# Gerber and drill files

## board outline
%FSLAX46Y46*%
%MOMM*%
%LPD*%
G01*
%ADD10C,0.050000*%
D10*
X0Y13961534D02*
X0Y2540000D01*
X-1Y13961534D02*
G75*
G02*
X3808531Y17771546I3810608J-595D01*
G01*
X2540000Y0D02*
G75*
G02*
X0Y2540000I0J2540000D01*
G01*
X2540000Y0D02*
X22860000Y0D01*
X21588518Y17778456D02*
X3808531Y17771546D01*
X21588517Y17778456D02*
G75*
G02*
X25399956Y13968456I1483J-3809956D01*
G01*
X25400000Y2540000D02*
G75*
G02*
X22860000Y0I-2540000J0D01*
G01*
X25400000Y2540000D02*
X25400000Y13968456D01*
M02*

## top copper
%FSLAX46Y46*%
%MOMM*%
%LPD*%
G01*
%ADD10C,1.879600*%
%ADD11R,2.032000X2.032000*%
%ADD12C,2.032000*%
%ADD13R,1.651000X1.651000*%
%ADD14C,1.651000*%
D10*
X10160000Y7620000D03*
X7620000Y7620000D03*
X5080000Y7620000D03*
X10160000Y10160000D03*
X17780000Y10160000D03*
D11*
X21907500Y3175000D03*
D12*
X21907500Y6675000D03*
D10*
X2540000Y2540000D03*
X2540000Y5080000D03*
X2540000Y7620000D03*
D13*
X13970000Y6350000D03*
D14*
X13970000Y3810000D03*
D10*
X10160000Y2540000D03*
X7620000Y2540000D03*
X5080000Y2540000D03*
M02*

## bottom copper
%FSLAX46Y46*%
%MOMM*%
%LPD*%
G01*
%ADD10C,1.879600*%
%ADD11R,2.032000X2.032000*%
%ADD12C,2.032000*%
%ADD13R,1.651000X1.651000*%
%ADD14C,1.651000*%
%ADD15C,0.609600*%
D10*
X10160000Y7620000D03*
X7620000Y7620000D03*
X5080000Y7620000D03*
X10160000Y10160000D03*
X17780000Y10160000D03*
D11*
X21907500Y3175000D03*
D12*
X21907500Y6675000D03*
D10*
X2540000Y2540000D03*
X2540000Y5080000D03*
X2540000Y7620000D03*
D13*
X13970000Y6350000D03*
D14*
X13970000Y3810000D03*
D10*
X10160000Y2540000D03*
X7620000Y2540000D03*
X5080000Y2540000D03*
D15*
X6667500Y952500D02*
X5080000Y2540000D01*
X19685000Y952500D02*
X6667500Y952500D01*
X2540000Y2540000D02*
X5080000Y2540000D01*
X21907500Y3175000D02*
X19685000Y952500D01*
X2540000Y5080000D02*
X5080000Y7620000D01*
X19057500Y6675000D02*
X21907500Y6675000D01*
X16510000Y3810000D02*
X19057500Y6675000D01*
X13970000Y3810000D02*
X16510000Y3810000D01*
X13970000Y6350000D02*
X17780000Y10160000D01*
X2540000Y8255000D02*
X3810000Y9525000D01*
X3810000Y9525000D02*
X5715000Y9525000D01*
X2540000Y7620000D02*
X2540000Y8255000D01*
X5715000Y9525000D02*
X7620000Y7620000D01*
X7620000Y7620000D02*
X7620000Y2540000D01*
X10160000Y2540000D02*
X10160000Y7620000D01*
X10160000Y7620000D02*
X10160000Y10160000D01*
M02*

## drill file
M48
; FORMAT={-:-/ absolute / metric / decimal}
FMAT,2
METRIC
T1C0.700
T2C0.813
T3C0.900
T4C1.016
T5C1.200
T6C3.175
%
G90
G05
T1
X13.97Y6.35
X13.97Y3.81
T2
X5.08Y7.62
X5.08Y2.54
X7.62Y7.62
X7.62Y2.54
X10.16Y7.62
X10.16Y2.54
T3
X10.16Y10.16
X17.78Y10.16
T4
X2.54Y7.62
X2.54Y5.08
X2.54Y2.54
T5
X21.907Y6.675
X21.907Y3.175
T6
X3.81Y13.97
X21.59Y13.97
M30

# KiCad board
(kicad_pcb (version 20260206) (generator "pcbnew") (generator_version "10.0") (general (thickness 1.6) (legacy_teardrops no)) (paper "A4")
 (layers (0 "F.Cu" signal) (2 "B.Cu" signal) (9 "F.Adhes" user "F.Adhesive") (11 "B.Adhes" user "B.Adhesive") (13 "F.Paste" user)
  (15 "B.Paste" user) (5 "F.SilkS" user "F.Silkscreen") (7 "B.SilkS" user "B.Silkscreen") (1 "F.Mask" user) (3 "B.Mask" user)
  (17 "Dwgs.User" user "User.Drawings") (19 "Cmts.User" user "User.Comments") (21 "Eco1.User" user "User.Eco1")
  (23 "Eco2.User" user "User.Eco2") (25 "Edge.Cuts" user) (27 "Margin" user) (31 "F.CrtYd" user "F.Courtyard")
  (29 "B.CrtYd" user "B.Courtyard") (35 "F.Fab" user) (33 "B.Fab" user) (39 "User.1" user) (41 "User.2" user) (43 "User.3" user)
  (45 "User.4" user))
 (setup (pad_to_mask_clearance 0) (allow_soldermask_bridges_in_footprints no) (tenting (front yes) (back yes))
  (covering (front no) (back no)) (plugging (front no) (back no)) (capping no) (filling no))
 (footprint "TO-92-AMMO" (layer "F.Cu") (at 7.62 -7.62 180)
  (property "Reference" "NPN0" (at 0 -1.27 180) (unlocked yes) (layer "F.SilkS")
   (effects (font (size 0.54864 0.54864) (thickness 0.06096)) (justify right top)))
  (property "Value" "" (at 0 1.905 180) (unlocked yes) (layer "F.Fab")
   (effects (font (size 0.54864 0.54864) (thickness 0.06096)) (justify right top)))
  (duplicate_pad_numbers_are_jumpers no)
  (pad "1" thru_hole circle (at -2.54 0 180) (size 1.8796 1.8796) (drill 0.8128) (layers "*.Cu" "*.Mask") (remove_unused_layers no)
   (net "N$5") (solder_mask_margin 0.1016) (thermal_bridge_angle 0))
  (pad "2" thru_hole circle (at 0 0 180) (size 1.8796 1.8796) (drill 0.8128) (layers "*.Cu" "*.Mask") (remove_unused_layers no) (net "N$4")
   (solder_mask_margin 0.1016) (thermal_bridge_angle 0))
  (pad "3" thru_hole circle (at 2.54 0 180) (size 1.8796 1.8796) (drill 0.8128) (layers "*.Cu" "*.Mask") (remove_unused_layers no)
   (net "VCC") (solder_mask_margin 0.1016) (thermal_bridge_angle 0)))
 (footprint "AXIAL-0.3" (layer "F.Cu") (at 13.97 -10.16)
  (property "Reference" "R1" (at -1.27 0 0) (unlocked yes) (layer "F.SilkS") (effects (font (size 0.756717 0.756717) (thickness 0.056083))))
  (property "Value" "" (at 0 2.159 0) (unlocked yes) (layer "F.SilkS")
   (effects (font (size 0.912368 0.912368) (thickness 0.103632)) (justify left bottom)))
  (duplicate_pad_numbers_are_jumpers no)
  (pad "P$1" thru_hole circle (at -3.81 0) (size 1.8796 1.8796) (drill 0.9) (layers "*.Cu" "*.Mask") (remove_unused_layers no) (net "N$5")
   (solder_mask_margin 0.1016) (thermal_bridge_angle 0))
  (pad "P$2" thru_hole circle (at 3.81 0) (size 1.8796 1.8796) (drill 0.9) (layers "*.Cu" "*.Mask") (remove_unused_layers no) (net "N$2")
   (solder_mask_margin 0.1016) (thermal_bridge_angle 0)))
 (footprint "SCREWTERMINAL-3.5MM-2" (layer "F.Cu") (at 21.9075 -3.175 90)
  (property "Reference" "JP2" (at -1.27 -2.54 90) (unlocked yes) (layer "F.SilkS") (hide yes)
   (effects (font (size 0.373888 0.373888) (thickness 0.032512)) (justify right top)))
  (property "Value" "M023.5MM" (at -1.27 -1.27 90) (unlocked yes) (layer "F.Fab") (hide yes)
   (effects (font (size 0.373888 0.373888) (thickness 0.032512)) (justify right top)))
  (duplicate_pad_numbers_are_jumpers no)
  (pad "1" thru_hole rect (at 0 0 90) (size 2.032 2.032) (drill 1.2) (layers "*.Cu" "*.Mask") (remove_unused_layers no) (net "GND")
   (solder_mask_margin 0.1016) (thermal_bridge_angle 0))
  (pad "2" thru_hole circle (at 3.5 0 90) (size 2.032 2.032) (drill 1.2) (layers "*.Cu" "*.Mask") (remove_unused_layers no) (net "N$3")
   (solder_mask_margin 0.1016) (thermal_bridge_angle 0)))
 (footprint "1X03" (layer "F.Cu") (at 2.54 -2.54 90)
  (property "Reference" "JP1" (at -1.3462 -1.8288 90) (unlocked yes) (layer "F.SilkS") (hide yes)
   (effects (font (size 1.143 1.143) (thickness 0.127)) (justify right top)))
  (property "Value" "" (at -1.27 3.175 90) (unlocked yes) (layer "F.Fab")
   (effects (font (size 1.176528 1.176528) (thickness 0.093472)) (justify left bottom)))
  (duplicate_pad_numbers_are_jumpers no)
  (pad "1" thru_hole circle (at 0 0 180) (size 1.8796 1.8796) (drill 1.016) (layers "*.Cu" "*.Mask") (remove_unused_layers no) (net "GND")
   (solder_mask_margin 0.1016) (thermal_bridge_angle 0))
  (pad "2" thru_hole circle (at 2.54 0 180) (size 1.8796 1.8796) (drill 1.016) (layers "*.Cu" "*.Mask") (remove_unused_layers no)
   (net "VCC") (solder_mask_margin 0.1016) (thermal_bridge_angle 0))
  (pad "3" thru_hole circle (at 5.08 0 180) (size 1.8796 1.8796) (drill 1.016) (layers "*.Cu" "*.Mask") (remove_unused_layers no)
   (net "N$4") (solder_mask_margin 0.1016) (thermal_bridge_angle 0)))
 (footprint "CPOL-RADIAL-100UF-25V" (layer "F.Cu") (at 13.97 -5.08 90)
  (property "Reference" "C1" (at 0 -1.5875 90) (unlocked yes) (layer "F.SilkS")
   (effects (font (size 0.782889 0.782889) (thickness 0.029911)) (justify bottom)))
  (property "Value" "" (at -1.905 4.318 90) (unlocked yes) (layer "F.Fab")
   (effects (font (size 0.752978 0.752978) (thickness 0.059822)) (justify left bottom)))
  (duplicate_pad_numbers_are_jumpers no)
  (pad "1" thru_hole rect (at 1.27 0 90) (size 1.651 1.651) (drill 0.7) (layers "*.Cu" "*.Mask") (remove_unused_layers no) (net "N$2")
   (solder_mask_margin 0.1016) (thermal_bridge_angle 0))
  (pad "2" thru_hole circle (at -1.27 0 90) (size 1.651 1.651) (drill 0.7) (layers "*.Cu" "*.Mask") (remove_unused_layers no) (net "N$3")
   (solder_mask_margin 0.1016) (thermal_bridge_angle 0)))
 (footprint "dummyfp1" (layer "F.Cu") (at 21.59 -13.97)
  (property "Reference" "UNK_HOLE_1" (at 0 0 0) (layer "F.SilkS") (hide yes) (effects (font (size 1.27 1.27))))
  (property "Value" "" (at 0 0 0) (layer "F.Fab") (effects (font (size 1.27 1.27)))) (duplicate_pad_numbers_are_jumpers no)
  (pad "" np_thru_hole circle (at 0 0) (size 3.175 3.175) (drill 3.175) (layers "*.Cu" "*.Mask")))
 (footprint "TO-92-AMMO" (layer "F.Cu") (at 7.62 -2.54 180)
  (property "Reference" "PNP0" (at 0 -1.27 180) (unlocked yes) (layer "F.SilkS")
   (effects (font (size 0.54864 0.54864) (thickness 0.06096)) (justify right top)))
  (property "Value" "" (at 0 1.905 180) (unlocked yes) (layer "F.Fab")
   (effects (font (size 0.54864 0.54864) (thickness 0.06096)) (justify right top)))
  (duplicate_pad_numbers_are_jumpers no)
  (pad "1" thru_hole circle (at -2.54 0 180) (size 1.8796 1.8796) (drill 0.8128) (layers "*.Cu" "*.Mask") (remove_unused_layers no)
   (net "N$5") (solder_mask_margin 0.1016) (thermal_bridge_angle 0))
  (pad "2" thru_hole circle (at 0 0 180) (size 1.8796 1.8796) (drill 0.8128) (layers "*.Cu" "*.Mask") (remove_unused_layers no) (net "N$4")
   (solder_mask_margin 0.1016) (thermal_bridge_angle 0))
  (pad "3" thru_hole circle (at 2.54 0 180) (size 1.8796 1.8796) (drill 0.8128) (layers "*.Cu" "*.Mask") (remove_unused_layers no)
   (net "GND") (solder_mask_margin 0.1016) (thermal_bridge_angle 0)))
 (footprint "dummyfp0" (layer "F.Cu") (at 3.81 -13.97)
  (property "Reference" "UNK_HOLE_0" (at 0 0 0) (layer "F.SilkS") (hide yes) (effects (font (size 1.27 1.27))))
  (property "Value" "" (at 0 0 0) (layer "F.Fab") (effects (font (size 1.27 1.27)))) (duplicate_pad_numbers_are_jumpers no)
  (pad "" np_thru_hole circle (at 0 0) (size 3.175 3.175) (drill 3.175) (layers "*.Cu" "*.Mask")))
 (gr_line (start 0 -13.961534) (end 0 -2.54) (stroke (width 0.05) (type solid)) (layer "Edge.Cuts"))
 (gr_arc (start -0.000001 -13.961534) (mid 1.115577 -16.654922) (end 3.808531 -17.771546) (stroke (width 0.05) (type solid))
  (layer "Edge.Cuts"))
 (gr_arc (start 2.54 0) (mid 0.743949 -0.743949) (end 0 -2.54) (stroke (width 0.05) (type solid)) (layer "Edge.Cuts"))
 (gr_line (start 2.54 0) (end 22.86 0) (stroke (width 0.05) (type solid)) (layer "Edge.Cuts"))
 (gr_line (start 21.588518 -17.778456) (end 3.808531 -17.771546) (stroke (width 0.05) (type solid)) (layer "Edge.Cuts"))
 (gr_arc (start 21.588517 -17.778456) (mid 24.283552 -16.663057) (end 25.4 -13.968456) (stroke (width 0.05) (type solid))
  (layer "Edge.Cuts"))
 (gr_arc (start 25.4 -2.54) (mid 24.656051 -0.743949) (end 22.86 0) (stroke (width 0.05) (type solid)) (layer "Edge.Cuts"))
 (gr_line (start 25.4 -2.54) (end 25.4 -13.968456) (stroke (width 0.05) (type solid)) (layer "Edge.Cuts"))
 (segment (start 6.6675 -0.9525) (end 5.08 -2.54) (width 0.6096) (layer "B.Cu") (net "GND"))
 (segment (start 19.685 -0.9525) (end 6.6675 -0.9525) (width 0.6096) (layer "B.Cu") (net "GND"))
 (segment (start 2.54 -2.54) (end 5.08 -2.54) (width 0.6096) (layer "B.Cu") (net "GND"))
 (segment (start 21.9075 -3.175) (end 19.685 -0.9525) (width 0.6096) (layer "B.Cu") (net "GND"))
 (segment (start 2.54 -5.08) (end 5.08 -7.62) (width 0.6096) (layer "B.Cu") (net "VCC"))
 (segment (start 19.0575 -6.675) (end 21.9075 -6.675) (width 0.6096) (layer "B.Cu") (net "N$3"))
 (segment (start 16.51 -3.81) (end 19.0575 -6.675) (width 0.6096) (layer "B.Cu") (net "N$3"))
 (segment (start 13.97 -3.81) (end 16.51 -3.81) (width 0.6096) (layer "B.Cu") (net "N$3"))
 (segment (start 13.97 -6.35) (end 17.78 -10.16) (width 0.6096) (layer "B.Cu") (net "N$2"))
 (segment (start 2.54 -8.255) (end 3.81 -9.525) (width 0.6096) (layer "B.Cu") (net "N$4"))
 (segment (start 3.81 -9.525) (end 5.715 -9.525) (width 0.6096) (layer "B.Cu") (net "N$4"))
 (segment (start 2.54 -7.62) (end 2.54 -8.255) (width 0.6096) (layer "B.Cu") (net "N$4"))
 (segment (start 5.715 -9.525) (end 7.62 -7.62) (width 0.6096) (layer "B.Cu") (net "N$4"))
 (segment (start 7.62 -7.62) (end 7.62 -2.54) (width 0.6096) (layer "B.Cu") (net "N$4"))
 (segment (start 10.16 -2.54) (end 10.16 -7.62) (width 0.6096) (layer "B.Cu") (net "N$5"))
 (segment (start 10.16 -7.62) (end 10.16 -10.16) (width 0.6096) (layer "B.Cu") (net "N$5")))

